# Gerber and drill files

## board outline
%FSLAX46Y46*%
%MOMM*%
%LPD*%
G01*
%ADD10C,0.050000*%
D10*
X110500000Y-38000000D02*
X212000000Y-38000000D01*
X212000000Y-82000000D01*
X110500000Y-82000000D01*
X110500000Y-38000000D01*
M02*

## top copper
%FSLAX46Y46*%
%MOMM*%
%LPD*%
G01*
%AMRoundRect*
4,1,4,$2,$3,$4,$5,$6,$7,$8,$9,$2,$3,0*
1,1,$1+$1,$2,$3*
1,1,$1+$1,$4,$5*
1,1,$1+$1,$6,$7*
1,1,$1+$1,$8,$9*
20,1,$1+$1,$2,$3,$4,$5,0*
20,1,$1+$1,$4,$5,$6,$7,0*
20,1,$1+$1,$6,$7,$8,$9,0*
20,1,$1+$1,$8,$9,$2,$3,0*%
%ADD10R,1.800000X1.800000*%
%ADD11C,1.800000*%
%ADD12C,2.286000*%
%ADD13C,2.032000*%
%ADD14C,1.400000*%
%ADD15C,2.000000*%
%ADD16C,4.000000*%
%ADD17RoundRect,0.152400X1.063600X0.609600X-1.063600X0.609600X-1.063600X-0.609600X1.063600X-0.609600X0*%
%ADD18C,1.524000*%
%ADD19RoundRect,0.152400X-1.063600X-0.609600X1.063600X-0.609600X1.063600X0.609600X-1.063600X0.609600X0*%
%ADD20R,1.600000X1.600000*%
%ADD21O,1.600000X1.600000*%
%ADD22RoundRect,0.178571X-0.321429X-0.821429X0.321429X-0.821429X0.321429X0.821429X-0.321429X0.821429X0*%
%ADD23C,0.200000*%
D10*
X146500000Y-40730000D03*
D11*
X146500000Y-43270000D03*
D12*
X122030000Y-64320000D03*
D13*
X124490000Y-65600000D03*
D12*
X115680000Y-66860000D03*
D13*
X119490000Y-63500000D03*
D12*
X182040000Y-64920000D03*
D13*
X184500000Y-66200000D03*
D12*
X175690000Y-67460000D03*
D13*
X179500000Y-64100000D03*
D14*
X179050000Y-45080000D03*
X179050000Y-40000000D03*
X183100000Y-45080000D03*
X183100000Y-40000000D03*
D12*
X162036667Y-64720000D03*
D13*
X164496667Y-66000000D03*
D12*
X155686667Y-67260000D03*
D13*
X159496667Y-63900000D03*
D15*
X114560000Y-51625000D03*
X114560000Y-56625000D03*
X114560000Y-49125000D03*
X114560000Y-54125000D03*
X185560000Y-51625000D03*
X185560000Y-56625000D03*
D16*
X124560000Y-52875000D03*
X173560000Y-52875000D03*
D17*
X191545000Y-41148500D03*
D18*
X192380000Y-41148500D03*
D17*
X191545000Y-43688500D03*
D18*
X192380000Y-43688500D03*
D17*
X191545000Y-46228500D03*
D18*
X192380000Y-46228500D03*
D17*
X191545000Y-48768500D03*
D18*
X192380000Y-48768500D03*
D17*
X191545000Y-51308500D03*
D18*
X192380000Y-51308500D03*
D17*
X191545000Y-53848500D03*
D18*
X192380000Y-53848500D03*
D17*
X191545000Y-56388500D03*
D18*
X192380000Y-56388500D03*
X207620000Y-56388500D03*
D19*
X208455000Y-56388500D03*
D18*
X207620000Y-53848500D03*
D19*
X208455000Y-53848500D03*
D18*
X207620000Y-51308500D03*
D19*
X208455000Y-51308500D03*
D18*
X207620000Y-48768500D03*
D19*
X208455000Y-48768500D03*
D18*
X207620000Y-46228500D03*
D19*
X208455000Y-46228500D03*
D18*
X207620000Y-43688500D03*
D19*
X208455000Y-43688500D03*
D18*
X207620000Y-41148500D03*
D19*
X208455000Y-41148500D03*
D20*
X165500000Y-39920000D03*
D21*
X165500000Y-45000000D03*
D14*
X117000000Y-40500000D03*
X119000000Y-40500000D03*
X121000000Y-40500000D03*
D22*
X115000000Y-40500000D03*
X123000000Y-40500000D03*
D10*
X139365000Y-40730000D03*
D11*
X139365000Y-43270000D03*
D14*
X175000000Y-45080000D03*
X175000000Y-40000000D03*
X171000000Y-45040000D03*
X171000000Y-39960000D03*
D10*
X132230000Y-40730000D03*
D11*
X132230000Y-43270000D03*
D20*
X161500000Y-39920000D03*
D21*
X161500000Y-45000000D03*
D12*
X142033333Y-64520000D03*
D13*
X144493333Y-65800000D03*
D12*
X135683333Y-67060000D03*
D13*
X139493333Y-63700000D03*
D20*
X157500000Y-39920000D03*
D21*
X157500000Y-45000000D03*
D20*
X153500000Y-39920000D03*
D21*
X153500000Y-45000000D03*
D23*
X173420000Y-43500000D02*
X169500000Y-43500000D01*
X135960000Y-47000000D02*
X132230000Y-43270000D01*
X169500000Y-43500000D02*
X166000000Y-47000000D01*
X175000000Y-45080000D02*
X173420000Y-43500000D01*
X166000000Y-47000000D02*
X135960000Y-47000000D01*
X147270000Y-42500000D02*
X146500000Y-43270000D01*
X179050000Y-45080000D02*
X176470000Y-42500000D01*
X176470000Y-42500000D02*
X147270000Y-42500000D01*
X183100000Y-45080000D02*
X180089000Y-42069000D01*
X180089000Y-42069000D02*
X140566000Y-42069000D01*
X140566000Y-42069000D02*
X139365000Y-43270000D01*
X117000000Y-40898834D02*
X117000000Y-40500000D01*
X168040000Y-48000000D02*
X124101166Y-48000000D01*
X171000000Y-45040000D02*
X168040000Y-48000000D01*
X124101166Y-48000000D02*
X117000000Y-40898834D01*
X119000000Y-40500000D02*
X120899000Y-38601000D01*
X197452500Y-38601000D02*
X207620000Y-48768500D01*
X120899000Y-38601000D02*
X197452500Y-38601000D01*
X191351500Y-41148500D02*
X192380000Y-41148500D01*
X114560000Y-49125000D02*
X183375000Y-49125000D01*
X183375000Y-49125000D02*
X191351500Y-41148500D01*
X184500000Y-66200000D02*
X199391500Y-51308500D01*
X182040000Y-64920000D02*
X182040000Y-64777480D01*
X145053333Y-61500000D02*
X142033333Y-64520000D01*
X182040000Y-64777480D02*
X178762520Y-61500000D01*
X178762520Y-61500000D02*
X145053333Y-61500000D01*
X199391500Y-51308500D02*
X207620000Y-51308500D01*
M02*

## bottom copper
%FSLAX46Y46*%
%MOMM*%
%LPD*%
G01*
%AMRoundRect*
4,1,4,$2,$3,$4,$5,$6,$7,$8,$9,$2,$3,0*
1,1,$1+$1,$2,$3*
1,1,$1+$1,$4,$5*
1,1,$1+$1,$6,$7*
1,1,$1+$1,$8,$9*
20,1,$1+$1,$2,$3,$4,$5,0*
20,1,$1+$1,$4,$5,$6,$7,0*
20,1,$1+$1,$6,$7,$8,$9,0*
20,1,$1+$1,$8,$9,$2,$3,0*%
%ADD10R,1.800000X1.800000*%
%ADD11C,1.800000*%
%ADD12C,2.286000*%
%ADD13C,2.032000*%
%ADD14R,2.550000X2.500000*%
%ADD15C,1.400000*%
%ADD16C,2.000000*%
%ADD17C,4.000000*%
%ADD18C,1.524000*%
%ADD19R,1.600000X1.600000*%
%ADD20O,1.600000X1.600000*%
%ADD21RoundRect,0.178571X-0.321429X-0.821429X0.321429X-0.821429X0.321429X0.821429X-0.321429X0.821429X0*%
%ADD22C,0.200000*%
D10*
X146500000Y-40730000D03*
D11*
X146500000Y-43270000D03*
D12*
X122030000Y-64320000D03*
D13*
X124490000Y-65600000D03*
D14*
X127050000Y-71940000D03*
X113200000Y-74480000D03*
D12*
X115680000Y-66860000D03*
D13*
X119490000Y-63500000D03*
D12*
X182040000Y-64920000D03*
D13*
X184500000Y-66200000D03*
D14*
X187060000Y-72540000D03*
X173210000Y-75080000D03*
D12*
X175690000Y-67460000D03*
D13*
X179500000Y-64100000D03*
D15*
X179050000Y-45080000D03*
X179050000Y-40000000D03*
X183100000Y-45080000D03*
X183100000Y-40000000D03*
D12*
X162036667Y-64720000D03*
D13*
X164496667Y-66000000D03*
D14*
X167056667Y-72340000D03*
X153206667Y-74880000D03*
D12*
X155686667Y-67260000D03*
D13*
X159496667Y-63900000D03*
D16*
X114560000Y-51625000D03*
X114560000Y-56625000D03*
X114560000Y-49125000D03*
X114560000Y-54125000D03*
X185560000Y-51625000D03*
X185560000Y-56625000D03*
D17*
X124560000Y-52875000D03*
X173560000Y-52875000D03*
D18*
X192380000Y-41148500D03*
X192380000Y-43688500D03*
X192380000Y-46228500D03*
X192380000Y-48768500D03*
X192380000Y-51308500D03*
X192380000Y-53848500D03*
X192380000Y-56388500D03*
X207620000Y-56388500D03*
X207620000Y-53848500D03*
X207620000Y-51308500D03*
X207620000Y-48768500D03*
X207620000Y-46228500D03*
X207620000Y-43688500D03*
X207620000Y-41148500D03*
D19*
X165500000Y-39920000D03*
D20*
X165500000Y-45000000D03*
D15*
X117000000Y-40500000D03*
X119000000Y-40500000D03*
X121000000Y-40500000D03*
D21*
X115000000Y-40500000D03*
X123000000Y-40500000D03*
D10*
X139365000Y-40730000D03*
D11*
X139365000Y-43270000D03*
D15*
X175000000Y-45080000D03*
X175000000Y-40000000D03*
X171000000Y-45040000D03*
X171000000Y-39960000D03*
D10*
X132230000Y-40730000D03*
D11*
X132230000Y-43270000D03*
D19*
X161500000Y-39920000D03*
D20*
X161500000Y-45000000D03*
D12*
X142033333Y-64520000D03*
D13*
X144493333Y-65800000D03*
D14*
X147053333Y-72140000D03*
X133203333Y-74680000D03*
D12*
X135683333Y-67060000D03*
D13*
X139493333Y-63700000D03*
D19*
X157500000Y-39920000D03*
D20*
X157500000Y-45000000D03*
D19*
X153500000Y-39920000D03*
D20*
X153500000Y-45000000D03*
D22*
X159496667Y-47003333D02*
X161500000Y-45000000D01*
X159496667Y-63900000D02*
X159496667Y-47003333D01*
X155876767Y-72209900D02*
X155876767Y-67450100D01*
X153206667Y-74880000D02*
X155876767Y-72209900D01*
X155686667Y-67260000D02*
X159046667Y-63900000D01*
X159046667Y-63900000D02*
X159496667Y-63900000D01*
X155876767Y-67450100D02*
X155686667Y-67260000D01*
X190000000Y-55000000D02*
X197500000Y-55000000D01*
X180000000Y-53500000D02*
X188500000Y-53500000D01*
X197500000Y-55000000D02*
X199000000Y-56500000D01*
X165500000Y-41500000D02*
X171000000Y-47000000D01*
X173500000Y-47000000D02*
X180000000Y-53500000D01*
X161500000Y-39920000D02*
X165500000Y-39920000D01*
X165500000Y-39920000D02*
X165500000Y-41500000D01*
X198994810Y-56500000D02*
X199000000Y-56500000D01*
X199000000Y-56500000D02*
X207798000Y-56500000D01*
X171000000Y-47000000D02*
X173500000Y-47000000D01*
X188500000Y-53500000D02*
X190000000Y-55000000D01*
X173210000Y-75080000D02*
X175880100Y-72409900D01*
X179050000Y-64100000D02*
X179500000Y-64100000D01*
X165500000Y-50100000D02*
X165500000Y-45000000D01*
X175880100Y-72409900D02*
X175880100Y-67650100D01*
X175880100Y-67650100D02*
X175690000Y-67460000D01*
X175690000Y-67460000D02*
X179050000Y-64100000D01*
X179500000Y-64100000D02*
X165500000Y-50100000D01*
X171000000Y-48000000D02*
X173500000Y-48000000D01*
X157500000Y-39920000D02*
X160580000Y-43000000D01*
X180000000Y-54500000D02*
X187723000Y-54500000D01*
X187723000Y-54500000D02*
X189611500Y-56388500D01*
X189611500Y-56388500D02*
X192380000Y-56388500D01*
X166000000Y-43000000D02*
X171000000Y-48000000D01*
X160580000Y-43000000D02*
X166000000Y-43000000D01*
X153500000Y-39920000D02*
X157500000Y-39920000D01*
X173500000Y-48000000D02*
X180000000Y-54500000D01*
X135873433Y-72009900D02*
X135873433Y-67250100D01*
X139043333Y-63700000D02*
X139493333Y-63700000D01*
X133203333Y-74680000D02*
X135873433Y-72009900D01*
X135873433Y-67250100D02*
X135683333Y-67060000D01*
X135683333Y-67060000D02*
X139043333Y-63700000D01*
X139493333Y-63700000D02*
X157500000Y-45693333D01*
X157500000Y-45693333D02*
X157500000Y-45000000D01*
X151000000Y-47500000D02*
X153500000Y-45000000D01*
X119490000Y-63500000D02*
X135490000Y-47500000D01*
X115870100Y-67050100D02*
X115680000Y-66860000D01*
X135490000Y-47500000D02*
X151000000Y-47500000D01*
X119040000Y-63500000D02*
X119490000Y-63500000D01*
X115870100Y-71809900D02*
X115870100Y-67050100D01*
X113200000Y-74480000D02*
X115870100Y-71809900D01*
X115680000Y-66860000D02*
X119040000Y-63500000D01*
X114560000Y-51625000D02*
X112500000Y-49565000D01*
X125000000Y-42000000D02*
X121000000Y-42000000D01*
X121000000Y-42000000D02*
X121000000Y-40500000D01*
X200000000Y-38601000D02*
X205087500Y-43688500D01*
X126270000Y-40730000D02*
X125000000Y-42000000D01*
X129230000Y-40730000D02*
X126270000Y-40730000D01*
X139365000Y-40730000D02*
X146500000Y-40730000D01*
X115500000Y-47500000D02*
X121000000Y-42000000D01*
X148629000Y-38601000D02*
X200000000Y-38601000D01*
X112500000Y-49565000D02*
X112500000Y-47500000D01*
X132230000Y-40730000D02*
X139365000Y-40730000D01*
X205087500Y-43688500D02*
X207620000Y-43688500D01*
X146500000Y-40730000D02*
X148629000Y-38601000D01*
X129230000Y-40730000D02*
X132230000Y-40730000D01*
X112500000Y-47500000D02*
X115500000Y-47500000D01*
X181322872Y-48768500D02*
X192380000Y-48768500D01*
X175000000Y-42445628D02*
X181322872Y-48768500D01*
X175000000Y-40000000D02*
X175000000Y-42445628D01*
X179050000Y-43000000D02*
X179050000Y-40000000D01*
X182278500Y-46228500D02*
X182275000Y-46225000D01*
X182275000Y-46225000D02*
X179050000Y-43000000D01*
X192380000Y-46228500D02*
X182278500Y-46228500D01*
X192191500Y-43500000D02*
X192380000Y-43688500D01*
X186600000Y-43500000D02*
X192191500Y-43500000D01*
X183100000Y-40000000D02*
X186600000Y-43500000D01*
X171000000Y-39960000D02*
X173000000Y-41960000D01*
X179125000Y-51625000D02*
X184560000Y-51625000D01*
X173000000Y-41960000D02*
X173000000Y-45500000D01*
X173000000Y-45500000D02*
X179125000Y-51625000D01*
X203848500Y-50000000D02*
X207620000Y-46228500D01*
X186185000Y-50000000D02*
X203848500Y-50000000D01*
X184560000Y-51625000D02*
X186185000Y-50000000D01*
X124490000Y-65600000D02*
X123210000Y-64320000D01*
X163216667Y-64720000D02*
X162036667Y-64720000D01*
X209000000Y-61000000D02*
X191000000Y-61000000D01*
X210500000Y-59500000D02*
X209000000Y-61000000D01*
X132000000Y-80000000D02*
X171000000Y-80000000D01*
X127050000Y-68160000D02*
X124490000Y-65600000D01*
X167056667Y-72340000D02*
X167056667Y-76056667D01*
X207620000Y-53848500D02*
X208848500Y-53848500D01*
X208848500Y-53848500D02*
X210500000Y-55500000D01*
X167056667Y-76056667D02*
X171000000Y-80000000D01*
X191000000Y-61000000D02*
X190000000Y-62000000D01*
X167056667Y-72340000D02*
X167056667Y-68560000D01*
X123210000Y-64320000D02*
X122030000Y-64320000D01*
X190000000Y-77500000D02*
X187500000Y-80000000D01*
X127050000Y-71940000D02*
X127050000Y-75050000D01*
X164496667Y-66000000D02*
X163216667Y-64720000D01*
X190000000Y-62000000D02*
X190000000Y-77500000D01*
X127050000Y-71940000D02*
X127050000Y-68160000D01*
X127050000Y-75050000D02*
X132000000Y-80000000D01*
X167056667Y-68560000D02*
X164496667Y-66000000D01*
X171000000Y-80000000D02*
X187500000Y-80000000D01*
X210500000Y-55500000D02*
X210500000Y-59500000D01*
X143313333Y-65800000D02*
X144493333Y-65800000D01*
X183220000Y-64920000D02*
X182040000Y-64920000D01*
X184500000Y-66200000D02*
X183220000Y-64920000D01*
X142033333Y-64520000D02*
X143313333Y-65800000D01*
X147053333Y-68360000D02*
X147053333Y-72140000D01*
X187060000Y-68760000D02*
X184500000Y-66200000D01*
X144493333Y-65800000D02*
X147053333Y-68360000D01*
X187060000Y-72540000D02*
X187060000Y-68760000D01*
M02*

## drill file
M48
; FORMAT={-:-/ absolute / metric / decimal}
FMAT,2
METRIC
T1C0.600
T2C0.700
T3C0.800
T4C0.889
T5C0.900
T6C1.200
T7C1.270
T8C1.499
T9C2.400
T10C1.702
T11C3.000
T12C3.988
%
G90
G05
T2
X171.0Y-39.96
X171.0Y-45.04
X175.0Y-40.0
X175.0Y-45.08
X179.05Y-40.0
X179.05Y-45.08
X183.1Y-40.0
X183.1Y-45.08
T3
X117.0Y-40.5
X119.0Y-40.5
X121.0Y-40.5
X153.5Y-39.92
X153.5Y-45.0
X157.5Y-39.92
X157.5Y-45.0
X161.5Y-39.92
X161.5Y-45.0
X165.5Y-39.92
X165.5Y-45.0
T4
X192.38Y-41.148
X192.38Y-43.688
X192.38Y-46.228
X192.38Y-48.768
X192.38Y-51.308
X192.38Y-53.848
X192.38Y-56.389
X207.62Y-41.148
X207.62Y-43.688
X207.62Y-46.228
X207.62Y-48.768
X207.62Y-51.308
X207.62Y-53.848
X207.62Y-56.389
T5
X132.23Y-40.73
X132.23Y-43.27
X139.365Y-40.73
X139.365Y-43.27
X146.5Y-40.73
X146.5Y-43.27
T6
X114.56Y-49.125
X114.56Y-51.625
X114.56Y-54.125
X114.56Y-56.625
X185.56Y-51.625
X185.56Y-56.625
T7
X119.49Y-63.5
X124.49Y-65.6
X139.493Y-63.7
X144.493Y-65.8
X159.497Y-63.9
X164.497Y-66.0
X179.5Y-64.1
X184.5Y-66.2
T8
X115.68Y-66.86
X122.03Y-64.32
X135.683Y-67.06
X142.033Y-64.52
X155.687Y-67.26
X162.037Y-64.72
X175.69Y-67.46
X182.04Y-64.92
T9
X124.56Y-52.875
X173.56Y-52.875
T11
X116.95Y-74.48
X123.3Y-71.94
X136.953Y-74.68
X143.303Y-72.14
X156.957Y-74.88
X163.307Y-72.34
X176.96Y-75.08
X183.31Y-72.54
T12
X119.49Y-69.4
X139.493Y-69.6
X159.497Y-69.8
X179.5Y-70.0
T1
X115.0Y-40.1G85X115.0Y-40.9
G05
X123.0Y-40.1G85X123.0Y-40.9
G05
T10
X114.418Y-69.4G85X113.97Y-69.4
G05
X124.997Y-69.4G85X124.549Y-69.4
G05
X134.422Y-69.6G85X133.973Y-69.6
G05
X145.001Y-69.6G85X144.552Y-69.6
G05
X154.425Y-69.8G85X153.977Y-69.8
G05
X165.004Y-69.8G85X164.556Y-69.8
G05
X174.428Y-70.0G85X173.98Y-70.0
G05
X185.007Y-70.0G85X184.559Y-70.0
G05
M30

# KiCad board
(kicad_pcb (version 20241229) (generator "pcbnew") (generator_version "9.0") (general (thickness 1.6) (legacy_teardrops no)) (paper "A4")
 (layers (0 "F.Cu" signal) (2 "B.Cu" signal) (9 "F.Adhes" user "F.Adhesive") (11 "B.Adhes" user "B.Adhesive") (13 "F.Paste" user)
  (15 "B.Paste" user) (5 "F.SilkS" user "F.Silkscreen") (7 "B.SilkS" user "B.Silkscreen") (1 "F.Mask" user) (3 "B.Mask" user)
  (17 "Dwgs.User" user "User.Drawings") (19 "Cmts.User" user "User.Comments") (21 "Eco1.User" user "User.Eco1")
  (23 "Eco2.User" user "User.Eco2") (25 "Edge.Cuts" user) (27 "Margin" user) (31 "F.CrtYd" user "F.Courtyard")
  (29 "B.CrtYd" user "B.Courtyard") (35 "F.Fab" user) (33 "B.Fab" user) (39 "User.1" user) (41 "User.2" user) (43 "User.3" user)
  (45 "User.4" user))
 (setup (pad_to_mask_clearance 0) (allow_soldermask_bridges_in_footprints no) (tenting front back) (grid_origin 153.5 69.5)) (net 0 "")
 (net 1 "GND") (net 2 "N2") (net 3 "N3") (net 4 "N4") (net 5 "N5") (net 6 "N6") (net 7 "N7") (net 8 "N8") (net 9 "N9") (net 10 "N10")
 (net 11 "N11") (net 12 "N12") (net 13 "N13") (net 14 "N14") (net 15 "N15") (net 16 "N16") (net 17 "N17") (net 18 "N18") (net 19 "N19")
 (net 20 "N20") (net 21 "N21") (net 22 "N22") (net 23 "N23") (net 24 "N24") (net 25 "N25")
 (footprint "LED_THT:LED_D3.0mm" (layer "F.Cu") (at 146.5 40.73 -90)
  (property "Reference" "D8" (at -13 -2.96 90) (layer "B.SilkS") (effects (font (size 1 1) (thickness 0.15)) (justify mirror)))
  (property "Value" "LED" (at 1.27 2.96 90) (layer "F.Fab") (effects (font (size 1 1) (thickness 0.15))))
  (pad "1" thru_hole rect (at 0 0 270) (size 1.8 1.8) (drill 0.9) (layers "*.Cu" "*.Mask") (remove_unused_layers no) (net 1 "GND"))
  (pad "2" thru_hole circle (at 2.54 0 270) (size 1.8 1.8) (drill 0.9) (layers "*.Cu" "*.Mask") (remove_unused_layers no) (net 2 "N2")))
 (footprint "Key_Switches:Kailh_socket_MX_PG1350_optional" (layer "F.Cu") (at 119.49 69.4)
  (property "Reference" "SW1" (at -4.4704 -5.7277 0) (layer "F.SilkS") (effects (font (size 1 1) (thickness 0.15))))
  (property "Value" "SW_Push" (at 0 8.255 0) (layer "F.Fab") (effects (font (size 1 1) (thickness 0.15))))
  (pad "" np_thru_hole oval (at -5.2959 0 180) (size 2.15 1.7018) (drill oval 2.15 1.7018) (layers "*.Cu" "*.Mask"))
  (pad "" np_thru_hole circle (at -2.54 5.08) (size 3 3) (drill 3) (layers "*.Cu" "*.Mask"))
  (pad "" np_thru_hole circle (at 0 0) (size 3.9878 3.9878) (drill 3.9878) (layers "*.Cu" "*.Mask"))
  (pad "" np_thru_hole circle (at 3.81 2.54) (size 3 3) (drill 3) (layers "*.Cu" "*.Mask"))
  (pad "" np_thru_hole oval (at 5.2832 0 180) (size 2.15 1.7018) (drill oval 2.15 1.7018) (layers "*.Cu" "*.Mask"))
  (pad "1" thru_hole circle (at 2.54 -5.08) (size 2.286 2.286) (drill 1.4986) (layers "*.Cu" "*.Mask") (remove_unused_layers no)
   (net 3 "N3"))
  (pad "1" thru_hole circle (at 5 -3.8 180) (size 2.032 2.032) (drill 1.27) (layers "*.Cu" "*.Mask") (remove_unused_layers no) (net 3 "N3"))
  (pad "1" smd rect (at 7.56 2.54) (size 2.55 2.5) (layers "B.Cu" "B.Mask" "B.Paste") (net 3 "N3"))
  (pad "2" smd rect (at -6.29 5.08) (size 2.55 2.5) (layers "B.Cu" "B.Mask" "B.Paste") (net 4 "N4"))
  (pad "2" thru_hole circle (at -3.81 -2.54) (size 2.286 2.286) (drill 1.4986) (layers "*.Cu" "*.Mask") (remove_unused_layers no)
   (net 4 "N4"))
  (pad "2" thru_hole circle (at 0 -5.9 180) (size 2.032 2.032) (drill 1.27) (layers "*.Cu" "*.Mask") (remove_unused_layers no) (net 4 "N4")))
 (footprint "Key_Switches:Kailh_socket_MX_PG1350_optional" (layer "F.Cu") (at 179.5 70)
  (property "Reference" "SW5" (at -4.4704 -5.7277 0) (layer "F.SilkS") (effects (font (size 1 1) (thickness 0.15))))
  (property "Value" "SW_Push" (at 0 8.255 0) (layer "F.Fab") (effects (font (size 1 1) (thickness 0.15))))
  (pad "" np_thru_hole oval (at -5.2959 0 180) (size 2.15 1.7018) (drill oval 2.15 1.7018) (layers "*.Cu" "*.Mask"))
  (pad "" np_thru_hole circle (at -2.54 5.08) (size 3 3) (drill 3) (layers "*.Cu" "*.Mask"))
  (pad "" np_thru_hole circle (at 0 0) (size 3.9878 3.9878) (drill 3.9878) (layers "*.Cu" "*.Mask"))
  (pad "" np_thru_hole circle (at 3.81 2.54) (size 3 3) (drill 3) (layers "*.Cu" "*.Mask"))
  (pad "" np_thru_hole oval (at 5.2832 0 180) (size 2.15 1.7018) (drill oval 2.15 1.7018) (layers "*.Cu" "*.Mask"))
  (pad "1" thru_hole circle (at 2.54 -5.08) (size 2.286 2.286) (drill 1.4986) (layers "*.Cu" "*.Mask") (remove_unused_layers no)
   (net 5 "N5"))
  (pad "1" thru_hole circle (at 5 -3.8 180) (size 2.032 2.032) (drill 1.27) (layers "*.Cu" "*.Mask") (remove_unused_layers no) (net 5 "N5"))
  (pad "1" smd rect (at 7.56 2.54) (size 2.55 2.5) (layers "B.Cu" "B.Mask" "B.Paste") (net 5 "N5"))
  (pad "2" smd rect (at -6.29 5.08) (size 2.55 2.5) (layers "B.Cu" "B.Mask" "B.Paste") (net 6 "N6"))
  (pad "2" thru_hole circle (at -3.81 -2.54) (size 2.286 2.286) (drill 1.4986) (layers "*.Cu" "*.Mask") (remove_unused_layers no)
   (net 6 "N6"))
  (pad "2" thru_hole circle (at 0 -5.9 180) (size 2.032 2.032) (drill 1.27) (layers "*.Cu" "*.Mask") (remove_unused_layers no) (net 6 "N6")))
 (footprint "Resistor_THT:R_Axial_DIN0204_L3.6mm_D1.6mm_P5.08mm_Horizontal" (layer "F.Cu") (at 179.05 45.08 90)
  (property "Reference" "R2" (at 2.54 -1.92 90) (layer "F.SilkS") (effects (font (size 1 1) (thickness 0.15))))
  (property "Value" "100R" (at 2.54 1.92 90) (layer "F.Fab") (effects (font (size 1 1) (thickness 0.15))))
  (pad "1" thru_hole circle (at 0 0 90) (size 1.4 1.4) (drill 0.7) (layers "*.Cu" "*.Mask") (remove_unused_layers no) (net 2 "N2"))
  (pad "2" thru_hole circle (at 5.08 0 90) (size 1.4 1.4) (drill 0.7) (layers "*.Cu" "*.Mask") (remove_unused_layers no) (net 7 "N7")))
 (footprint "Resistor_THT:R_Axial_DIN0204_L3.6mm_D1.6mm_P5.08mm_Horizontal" (layer "F.Cu") (at 183.1 45.08 90)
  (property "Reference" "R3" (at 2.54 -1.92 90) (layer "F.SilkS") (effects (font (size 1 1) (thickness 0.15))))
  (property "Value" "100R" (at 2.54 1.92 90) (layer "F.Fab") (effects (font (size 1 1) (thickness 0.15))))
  (pad "1" thru_hole circle (at 0 0 90) (size 1.4 1.4) (drill 0.7) (layers "*.Cu" "*.Mask") (remove_unused_layers no) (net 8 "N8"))
  (pad "2" thru_hole circle (at 5.08 0 90) (size 1.4 1.4) (drill 0.7) (layers "*.Cu" "*.Mask") (remove_unused_layers no) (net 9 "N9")))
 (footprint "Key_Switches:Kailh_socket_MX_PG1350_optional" (layer "F.Cu") (at 159.496667 69.8)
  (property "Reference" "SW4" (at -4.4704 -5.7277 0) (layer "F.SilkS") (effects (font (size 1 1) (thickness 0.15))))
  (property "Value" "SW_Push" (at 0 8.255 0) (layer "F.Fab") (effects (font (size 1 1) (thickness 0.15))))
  (pad "" np_thru_hole oval (at -5.2959 0 180) (size 2.15 1.7018) (drill oval 2.15 1.7018) (layers "*.Cu" "*.Mask"))
  (pad "" np_thru_hole circle (at -2.54 5.08) (size 3 3) (drill 3) (layers "*.Cu" "*.Mask"))
  (pad "" np_thru_hole circle (at 0 0) (size 3.9878 3.9878) (drill 3.9878) (layers "*.Cu" "*.Mask"))
  (pad "" np_thru_hole circle (at 3.81 2.54) (size 3 3) (drill 3) (layers "*.Cu" "*.Mask"))
  (pad "" np_thru_hole oval (at 5.2832 0 180) (size 2.15 1.7018) (drill oval 2.15 1.7018) (layers "*.Cu" "*.Mask"))
  (pad "1" thru_hole circle (at 2.54 -5.08) (size 2.286 2.286) (drill 1.4986) (layers "*.Cu" "*.Mask") (remove_unused_layers no)
   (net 3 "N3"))
  (pad "1" thru_hole circle (at 5 -3.8 180) (size 2.032 2.032) (drill 1.27) (layers "*.Cu" "*.Mask") (remove_unused_layers no) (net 3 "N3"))
  (pad "1" smd rect (at 7.56 2.54) (size 2.55 2.5) (layers "B.Cu" "B.Mask" "B.Paste") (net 3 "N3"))
  (pad "2" smd rect (at -6.29 5.08) (size 2.55 2.5) (layers "B.Cu" "B.Mask" "B.Paste") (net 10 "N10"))
  (pad "2" thru_hole circle (at -3.81 -2.54) (size 2.286 2.286) (drill 1.4986) (layers "*.Cu" "*.Mask") (remove_unused_layers no)
   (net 10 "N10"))
  (pad "2" thru_hole circle (at 0 -5.9 180) (size 2.032 2.032) (drill 1.27) (layers "*.Cu" "*.Mask") (remove_unused_layers no)
   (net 10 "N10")))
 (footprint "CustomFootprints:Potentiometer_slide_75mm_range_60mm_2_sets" (layer "F.Cu") (at 112.06 57.625)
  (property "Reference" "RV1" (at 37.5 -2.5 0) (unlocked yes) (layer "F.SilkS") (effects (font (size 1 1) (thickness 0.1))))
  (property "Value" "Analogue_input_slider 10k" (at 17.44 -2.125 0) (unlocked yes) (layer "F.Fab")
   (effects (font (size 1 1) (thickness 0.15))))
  (pad "1" thru_hole circle (at 2.5 -6) (size 2 2) (drill 1.2) (layers "*.Cu" "*.Mask") (remove_unused_layers no) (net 1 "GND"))
  (pad "1'" thru_hole circle (at 2.5 -1) (size 2 2) (drill 1.2) (layers "*.Cu" "*.Mask") (remove_unused_layers no))
  (pad "2" thru_hole circle (at 2.5 -8.5) (size 2 2) (drill 1.2) (layers "*.Cu" "*.Mask") (remove_unused_layers no) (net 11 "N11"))
  (pad "2'" thru_hole circle (at 2.5 -3.5) (size 2 2) (drill 1.2) (layers "*.Cu" "*.Mask") (remove_unused_layers no))
  (pad "3" thru_hole circle (at 73.5 -6) (size 2 2) (drill 1.2) (layers "*.Cu" "*.Mask") (remove_unused_layers no) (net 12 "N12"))
  (pad "3'" thru_hole circle (at 73.5 -1) (size 2 2) (drill 1.2) (layers "*.Cu" "*.Mask") (remove_unused_layers no))
  (pad "MP" thru_hole circle (at 12.5 -4.75) (size 4 4) (drill 2.4) (layers "*.Cu" "*.Mask") (remove_unused_layers no))
  (pad "MP" thru_hole circle (at 61.5 -4.75) (size 4 4) (drill 2.4) (layers "*.Cu" "*.Mask") (remove_unused_layers no)))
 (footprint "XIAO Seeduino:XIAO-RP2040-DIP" (layer "F.Cu") (at 200 48.7685)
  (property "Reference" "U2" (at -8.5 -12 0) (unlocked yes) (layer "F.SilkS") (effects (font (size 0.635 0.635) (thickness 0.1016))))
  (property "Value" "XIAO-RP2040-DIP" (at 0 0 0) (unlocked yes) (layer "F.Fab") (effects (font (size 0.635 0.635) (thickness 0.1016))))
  (pad "1" smd roundrect (at -8.455 -7.62 180) (size 2.432 1.524) (layers "F.Cu" "F.Mask") (roundrect_rratio 0.1) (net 11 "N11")
   (thermal_bridge_angle 45))
  (pad "1" thru_hole circle (at -7.62 -7.62 180) (size 1.524 1.524) (drill 0.889) (layers "*.Cu" "*.Mask") (remove_unused_layers no)
   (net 11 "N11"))
  (pad "2" smd roundrect (at -8.455 -5.08 180) (size 2.432 1.524) (layers "F.Cu" "F.Mask") (roundrect_rratio 0.1) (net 9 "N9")
   (thermal_bridge_angle 45))
  (pad "2" thru_hole circle (at -7.62 -5.08 180) (size 1.524 1.524) (drill 0.889) (layers "*.Cu" "*.Mask") (remove_unused_layers no)
   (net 9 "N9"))
  (pad "3" smd roundrect (at -8.455 -2.54 180) (size 2.432 1.524) (layers "F.Cu" "F.Mask") (roundrect_rratio 0.1) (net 7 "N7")
   (thermal_bridge_angle 45))
  (pad "3" thru_hole circle (at -7.62 -2.54 180) (size 1.524 1.524) (drill 0.889) (layers "*.Cu" "*.Mask") (remove_unused_layers no)
   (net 7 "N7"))
  (pad "4" smd roundrect (at -8.455 0 180) (size 2.432 1.524) (layers "F.Cu" "F.Mask") (roundrect_rratio 0.1) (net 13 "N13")
   (thermal_bridge_angle 45))
  (pad "4" thru_hole circle (at -7.62 0 180) (size 1.524 1.524) (drill 0.889) (layers "*.Cu" "*.Mask") (remove_unused_layers no)
   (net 13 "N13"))
  (pad "5" smd roundrect (at -8.455 2.54 180) (size 2.432 1.524) (layers "F.Cu" "F.Mask") (roundrect_rratio 0.1) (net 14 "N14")
   (thermal_bridge_angle 45))
  (pad "5" thru_hole circle (at -7.62 2.54 180) (size 1.524 1.524) (drill 0.889) (layers "*.Cu" "*.Mask") (remove_unused_layers no)
   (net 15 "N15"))
  (pad "6" smd roundrect (at -8.455 5.08 180) (size 2.432 1.524) (layers "F.Cu" "F.Mask") (roundrect_rratio 0.1) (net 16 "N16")
   (thermal_bridge_angle 45))
  (pad "6" thru_hole circle (at -7.62 5.08 180) (size 1.524 1.524) (drill 0.889) (layers "*.Cu" "*.Mask") (remove_unused_layers no)
   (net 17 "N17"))
  (pad "7" smd roundrect (at -8.455 7.62 180) (size 2.432 1.524) (layers "F.Cu" "F.Mask") (roundrect_rratio 0.1) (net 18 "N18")
   (thermal_bridge_angle 45))
  (pad "7" thru_hole circle (at -7.62 7.62 180) (size 1.524 1.524) (drill 0.889) (layers "*.Cu" "*.Mask") (remove_unused_layers no)
   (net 18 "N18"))
  (pad "8" thru_hole circle (at 7.62 7.62) (size 1.524 1.524) (drill 0.889) (layers "*.Cu" "*.Mask") (remove_unused_layers no)
   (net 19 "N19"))
  (pad "8" smd roundrect (at 8.455 7.62) (size 2.432 1.524) (layers "F.Cu" "F.Mask") (roundrect_rratio 0.1) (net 19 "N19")
   (thermal_bridge_angle 45))
  (pad "9" thru_hole circle (at 7.62 5.08) (size 1.524 1.524) (drill 0.889) (layers "*.Cu" "*.Mask") (remove_unused_layers no) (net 3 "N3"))
  (pad "9" smd roundrect (at 8.455 5.08) (size 2.432 1.524) (layers "F.Cu" "F.Mask") (roundrect_rratio 0.1) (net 3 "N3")
   (thermal_bridge_angle 45))
  (pad "10" thru_hole circle (at 7.62 2.54) (size 1.524 1.524) (drill 0.889) (layers "*.Cu" "*.Mask") (remove_unused_layers no) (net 5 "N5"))
  (pad "10" smd roundrect (at 8.455 2.54) (size 2.432 1.524) (layers "F.Cu" "F.Mask") (roundrect_rratio 0.1) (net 5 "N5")
   (thermal_bridge_angle 45))
  (pad "11" thru_hole circle (at 7.62 0) (size 1.524 1.524) (drill 0.889) (layers "*.Cu" "*.Mask") (remove_unused_layers no) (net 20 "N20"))
  (pad "11" smd roundrect (at 8.455 0) (size 2.432 1.524) (layers "F.Cu" "F.Mask") (roundrect_rratio 0.1) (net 20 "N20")
   (thermal_bridge_angle 45))
  (pad "12" thru_hole circle (at 7.62 -2.54) (size 1.524 1.524) (drill 0.889) (layers "*.Cu" "*.Mask") (remove_unused_layers no)
   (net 12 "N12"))
  (pad "12" smd roundrect (at 8.455 -2.54) (size 2.432 1.524) (layers "F.Cu" "F.Mask") (roundrect_rratio 0.1) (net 12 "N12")
   (thermal_bridge_angle 45))
  (pad "13" thru_hole circle (at 7.62 -5.08) (size 1.524 1.524) (drill 0.889) (layers "*.Cu" "*.Mask") (remove_unused_layers no)
   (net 1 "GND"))
  (pad "13" smd roundrect (at 8.455 -5.08) (size 2.432 1.524) (layers "F.Cu" "F.Mask") (roundrect_rratio 0.1) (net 1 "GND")
   (thermal_bridge_angle 45))
  (pad "14" thru_hole circle (at 7.62 -7.62) (size 1.524 1.524) (drill 0.889) (layers "*.Cu" "*.Mask") (remove_unused_layers no)
   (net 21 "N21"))
  (pad "14" smd roundrect (at 8.455 -7.62) (size 2.432 1.524) (layers "F.Cu" "F.Mask") (roundrect_rratio 0.1) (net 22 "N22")
   (thermal_bridge_angle 45)))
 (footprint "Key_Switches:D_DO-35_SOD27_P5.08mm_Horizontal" (layer "F.Cu") (at 165.5 38.65 -90)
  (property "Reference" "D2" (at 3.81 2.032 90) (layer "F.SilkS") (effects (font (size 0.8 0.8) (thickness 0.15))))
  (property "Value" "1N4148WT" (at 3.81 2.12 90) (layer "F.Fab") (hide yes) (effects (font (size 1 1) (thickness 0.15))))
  (pad "1" thru_hole rect (at 1.27 0 270) (size 1.6 1.6) (drill 0.8) (layers "*.Cu" "*.Mask") (remove_unused_layers no) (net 19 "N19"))
  (pad "2" thru_hole oval (at 6.35 0 270) (size 1.6 1.6) (drill 0.8) (layers "*.Cu" "*.Mask") (remove_unused_layers no) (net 6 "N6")))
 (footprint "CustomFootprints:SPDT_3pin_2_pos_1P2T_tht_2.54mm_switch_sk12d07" (layer "F.Cu") (at 114.7 38.25)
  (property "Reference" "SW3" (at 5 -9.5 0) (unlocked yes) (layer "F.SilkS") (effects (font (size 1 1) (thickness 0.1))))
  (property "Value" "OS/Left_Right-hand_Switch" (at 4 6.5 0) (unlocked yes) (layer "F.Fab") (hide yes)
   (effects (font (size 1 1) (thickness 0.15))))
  (pad "1" thru_hole circle (at 2.3 2.25) (size 1.4 1.4) (drill 0.8) (layers "*.Cu" "*.Mask") (remove_unused_layers no) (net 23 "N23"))
  (pad "2" thru_hole circle (at 4.3 2.25) (size 1.4 1.4) (drill 0.8) (layers "*.Cu" "*.Mask") (remove_unused_layers no) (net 20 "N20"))
  (pad "3" thru_hole circle (at 6.3 2.25) (size 1.4 1.4) (drill 0.8) (layers "*.Cu" "*.Mask") (remove_unused_layers no) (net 1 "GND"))
  (pad "MH" thru_hole roundrect (at 0.3 2.25) (size 1 2) (drill oval 0.6 1.4) (layers "*.Cu" "*.Mask") (remove_unused_layers no)
   (roundrect_rratio 0.1785714286))
  (pad "MH" thru_hole roundrect (at 8.3 2.25) (size 1 2) (drill oval 0.6 1.4) (layers "*.Cu" "*.Mask") (remove_unused_layers no)
   (roundrect_rratio 0.1785714286)))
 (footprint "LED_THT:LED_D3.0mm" (layer "F.Cu") (at 139.365 40.73 -90)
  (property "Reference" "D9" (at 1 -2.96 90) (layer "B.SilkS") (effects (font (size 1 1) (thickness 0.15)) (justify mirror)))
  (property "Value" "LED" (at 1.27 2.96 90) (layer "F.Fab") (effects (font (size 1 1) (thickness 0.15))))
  (pad "1" thru_hole rect (at 0 0 270) (size 1.8 1.8) (drill 0.9) (layers "*.Cu" "*.Mask") (remove_unused_layers no) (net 1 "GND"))
  (pad "2" thru_hole circle (at 2.54 0 270) (size 1.8 1.8) (drill 0.9) (layers "*.Cu" "*.Mask") (remove_unused_layers no) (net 8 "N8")))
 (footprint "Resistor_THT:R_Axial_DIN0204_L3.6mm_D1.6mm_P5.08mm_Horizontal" (layer "F.Cu") (at 175 45.08 90)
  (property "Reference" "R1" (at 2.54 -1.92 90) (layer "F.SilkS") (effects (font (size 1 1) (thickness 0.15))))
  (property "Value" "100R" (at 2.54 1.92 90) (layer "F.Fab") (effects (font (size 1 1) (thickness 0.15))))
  (pad "1" thru_hole circle (at 0 0 90) (size 1.4 1.4) (drill 0.7) (layers "*.Cu" "*.Mask") (remove_unused_layers no) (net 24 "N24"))
  (pad "2" thru_hole circle (at 5.08 0 90) (size 1.4 1.4) (drill 0.7) (layers "*.Cu" "*.Mask") (remove_unused_layers no) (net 13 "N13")))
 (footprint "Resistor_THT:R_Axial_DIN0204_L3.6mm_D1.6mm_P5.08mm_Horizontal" (layer "F.Cu") (at 171 45.04 90)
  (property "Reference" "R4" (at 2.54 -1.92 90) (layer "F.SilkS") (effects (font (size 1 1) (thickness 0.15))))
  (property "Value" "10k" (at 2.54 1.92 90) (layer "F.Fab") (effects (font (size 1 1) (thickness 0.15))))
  (pad "1" thru_hole circle (at 0 0 90) (size 1.4 1.4) (drill 0.7) (layers "*.Cu" "*.Mask") (remove_unused_layers no) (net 23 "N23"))
  (pad "2" thru_hole circle (at 5.08 0 90) (size 1.4 1.4) (drill 0.7) (layers "*.Cu" "*.Mask") (remove_unused_layers no) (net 12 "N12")))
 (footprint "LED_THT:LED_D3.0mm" (layer "F.Cu") (at 132.23 40.73 -90)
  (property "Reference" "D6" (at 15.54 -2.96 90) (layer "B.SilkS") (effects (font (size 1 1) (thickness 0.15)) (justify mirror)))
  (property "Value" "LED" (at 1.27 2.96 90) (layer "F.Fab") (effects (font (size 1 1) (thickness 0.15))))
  (pad "1" thru_hole rect (at 0 0 270) (size 1.8 1.8) (drill 0.9) (layers "*.Cu" "*.Mask") (remove_unused_layers no) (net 1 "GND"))
  (pad "2" thru_hole circle (at 2.54 0 270) (size 1.8 1.8) (drill 0.9) (layers "*.Cu" "*.Mask") (remove_unused_layers no) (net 24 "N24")))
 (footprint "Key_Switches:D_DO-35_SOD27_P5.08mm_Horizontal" (layer "F.Cu") (at 161.5 38.65 -90)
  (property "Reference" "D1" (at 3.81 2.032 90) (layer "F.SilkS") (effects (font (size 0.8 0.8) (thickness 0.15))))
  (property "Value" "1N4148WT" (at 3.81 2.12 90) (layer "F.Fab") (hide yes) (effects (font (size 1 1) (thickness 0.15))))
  (pad "1" thru_hole rect (at 1.27 0 270) (size 1.6 1.6) (drill 0.8) (layers "*.Cu" "*.Mask") (remove_unused_layers no) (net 19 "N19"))
  (pad "2" thru_hole oval (at 6.35 0 270) (size 1.6 1.6) (drill 0.8) (layers "*.Cu" "*.Mask") (remove_unused_layers no) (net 10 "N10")))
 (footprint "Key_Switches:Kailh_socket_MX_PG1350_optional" (layer "F.Cu") (at 139.493333 69.6)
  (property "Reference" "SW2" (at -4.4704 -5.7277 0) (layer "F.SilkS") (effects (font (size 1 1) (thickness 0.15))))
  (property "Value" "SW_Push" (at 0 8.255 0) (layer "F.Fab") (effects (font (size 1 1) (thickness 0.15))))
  (pad "" np_thru_hole oval (at -5.2959 0 180) (size 2.15 1.7018) (drill oval 2.15 1.7018) (layers "*.Cu" "*.Mask"))
  (pad "" np_thru_hole circle (at -2.54 5.08) (size 3 3) (drill 3) (layers "*.Cu" "*.Mask"))
  (pad "" np_thru_hole circle (at 0 0) (size 3.9878 3.9878) (drill 3.9878) (layers "*.Cu" "*.Mask"))
  (pad "" np_thru_hole circle (at 3.81 2.54) (size 3 3) (drill 3) (layers "*.Cu" "*.Mask"))
  (pad "" np_thru_hole oval (at 5.2832 0 180) (size 2.15 1.7018) (drill oval 2.15 1.7018) (layers "*.Cu" "*.Mask"))
  (pad "1" thru_hole circle (at 2.54 -5.08) (size 2.286 2.286) (drill 1.4986) (layers "*.Cu" "*.Mask") (remove_unused_layers no)
   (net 5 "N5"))
  (pad "1" thru_hole circle (at 5 -3.8 180) (size 2.032 2.032) (drill 1.27) (layers "*.Cu" "*.Mask") (remove_unused_layers no) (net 5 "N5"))
  (pad "1" smd rect (at 7.56 2.54) (size 2.55 2.5) (layers "B.Cu" "B.Mask" "B.Paste") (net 5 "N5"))
  (pad "2" smd rect (at -6.29 5.08) (size 2.55 2.5) (layers "B.Cu" "B.Mask" "B.Paste") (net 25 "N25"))
  (pad "2" thru_hole circle (at -3.81 -2.54) (size 2.286 2.286) (drill 1.4986) (layers "*.Cu" "*.Mask") (remove_unused_layers no)
   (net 25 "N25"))
  (pad "2" thru_hole circle (at 0 -5.9 180) (size 2.032 2.032) (drill 1.27) (layers "*.Cu" "*.Mask") (remove_unused_layers no)
   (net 25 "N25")))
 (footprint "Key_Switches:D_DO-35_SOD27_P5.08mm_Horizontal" (layer "F.Cu") (at 157.5 38.65 -90)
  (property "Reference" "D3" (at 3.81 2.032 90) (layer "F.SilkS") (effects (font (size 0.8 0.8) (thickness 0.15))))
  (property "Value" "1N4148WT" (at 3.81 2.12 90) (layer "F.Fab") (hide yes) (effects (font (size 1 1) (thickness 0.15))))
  (pad "1" thru_hole rect (at 1.27 0 270) (size 1.6 1.6) (drill 0.8) (layers "*.Cu" "*.Mask") (remove_unused_layers no) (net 18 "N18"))
  (pad "2" thru_hole oval (at 6.35 0 270) (size 1.6 1.6) (drill 0.8) (layers "*.Cu" "*.Mask") (remove_unused_layers no) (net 25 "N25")))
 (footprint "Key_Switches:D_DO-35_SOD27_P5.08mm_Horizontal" (layer "F.Cu") (at 153.5 38.65 -90)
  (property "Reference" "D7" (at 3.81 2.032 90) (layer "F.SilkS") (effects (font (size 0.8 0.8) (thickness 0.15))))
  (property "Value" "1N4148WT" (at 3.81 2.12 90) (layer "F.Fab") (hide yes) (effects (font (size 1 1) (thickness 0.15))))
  (pad "1" thru_hole rect (at 1.27 0 270) (size 1.6 1.6) (drill 0.8) (layers "*.Cu" "*.Mask") (remove_unused_layers no) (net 18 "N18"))
  (pad "2" thru_hole oval (at 6.35 0 270) (size 1.6 1.6) (drill 0.8) (layers "*.Cu" "*.Mask") (remove_unused_layers no) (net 4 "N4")))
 (gr_rect (start 110.5 38) (end 212 82) (stroke (width 0.05) (type default)) (fill no) (layer "Edge.Cuts"))
 (segment (start 159.496667 47.003333) (end 161.5 45) (width 0.2) (layer "B.Cu") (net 10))
 (segment (start 159.496667 63.9) (end 159.496667 47.003333) (width 0.2) (layer "B.Cu") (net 10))
 (segment (start 155.876767 72.2099) (end 155.876767 67.4501) (width 0.2) (layer "B.Cu") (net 10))
 (segment (start 153.206667 74.88) (end 155.876767 72.2099) (width 0.2) (layer "B.Cu") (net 10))
 (segment (start 155.686667 67.26) (end 159.046667 63.9) (width 0.2) (layer "B.Cu") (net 10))
 (segment (start 159.046667 63.9) (end 159.496667 63.9) (width 0.2) (layer "B.Cu") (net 10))
 (segment (start 155.876767 67.4501) (end 155.686667 67.26) (width 0.2) (layer "B.Cu") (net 10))
 (segment (start 190 55) (end 197.5 55) (width 0.2) (layer "B.Cu") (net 19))
 (segment (start 180 53.5) (end 188.5 53.5) (width 0.2) (layer "B.Cu") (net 19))
 (segment (start 197.5 55) (end 199 56.5) (width 0.2) (layer "B.Cu") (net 19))
 (segment (start 165.5 41.5) (end 171 47) (width 0.2) (layer "B.Cu") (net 19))
 (segment (start 173.5 47) (end 180 53.5) (width 0.2) (layer "B.Cu") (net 19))
 (segment (start 161.5 39.92) (end 165.5 39.92) (width 0.2) (layer "B.Cu") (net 19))
 (segment (start 165.5 39.92) (end 165.5 41.5) (width 0.2) (layer "B.Cu") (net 19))
 (segment (start 198.99481 56.5) (end 199 56.5) (width 0.2) (layer "B.Cu") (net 19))
 (segment (start 199 56.5) (end 207.798 56.5) (width 0.2) (layer "B.Cu") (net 19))
 (segment (start 171 47) (end 173.5 47) (width 0.2) (layer "B.Cu") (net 19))
 (segment (start 188.5 53.5) (end 190 55) (width 0.2) (layer "B.Cu") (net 19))
 (segment (start 173.21 75.08) (end 175.8801 72.4099) (width 0.2) (layer "B.Cu") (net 6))
 (segment (start 179.05 64.1) (end 179.5 64.1) (width 0.2) (layer "B.Cu") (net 6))
 (segment (start 165.5 50.1) (end 165.5 45) (width 0.2) (layer "B.Cu") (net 6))
 (segment (start 175.8801 72.4099) (end 175.8801 67.6501) (width 0.2) (layer "B.Cu") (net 6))
 (segment (start 175.8801 67.6501) (end 175.69 67.46) (width 0.2) (layer "B.Cu") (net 6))
 (segment (start 175.69 67.46) (end 179.05 64.1) (width 0.2) (layer "B.Cu") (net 6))
 (segment (start 179.5 64.1) (end 165.5 50.1) (width 0.2) (layer "B.Cu") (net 6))
 (segment (start 171 48) (end 173.5 48) (width 0.2) (layer "B.Cu") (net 18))
 (segment (start 157.5 39.92) (end 160.58 43) (width 0.2) (layer "B.Cu") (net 18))
 (segment (start 180 54.5) (end 187.723 54.5) (width 0.2) (layer "B.Cu") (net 18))
 (segment (start 187.723 54.5) (end 189.6115 56.3885) (width 0.2) (layer "B.Cu") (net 18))
 (segment (start 189.6115 56.3885) (end 192.38 56.3885) (width 0.2) (layer "B.Cu") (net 18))
 (segment (start 166 43) (end 171 48) (width 0.2) (layer "B.Cu") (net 18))
 (segment (start 160.58 43) (end 166 43) (width 0.2) (layer "B.Cu") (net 18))
 (segment (start 153.5 39.92) (end 157.5 39.92) (width 0.2) (layer "B.Cu") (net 18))
 (segment (start 173.5 48) (end 180 54.5) (width 0.2) (layer "B.Cu") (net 18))
 (segment (start 135.873433 72.0099) (end 135.873433 67.2501) (width 0.2) (layer "B.Cu") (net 25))
 (segment (start 139.043333 63.7) (end 139.493333 63.7) (width 0.2) (layer "B.Cu") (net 25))
 (segment (start 133.203333 74.68) (end 135.873433 72.0099) (width 0.2) (layer "B.Cu") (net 25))
 (segment (start 135.873433 67.2501) (end 135.683333 67.06) (width 0.2) (layer "B.Cu") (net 25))
 (segment (start 135.683333 67.06) (end 139.043333 63.7) (width 0.2) (layer "B.Cu") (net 25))
 (segment (start 139.493333 63.7) (end 157.5 45.693333) (width 0.2) (layer "B.Cu") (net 25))
 (segment (start 157.5 45.693333) (end 157.5 45) (width 0.2) (layer "B.Cu") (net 25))
 (segment (start 151 47.5) (end 153.5 45) (width 0.2) (layer "B.Cu") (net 4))
 (segment (start 119.49 63.5) (end 135.49 47.5) (width 0.2) (layer "B.Cu") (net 4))
 (segment (start 115.8701 67.0501) (end 115.68 66.86) (width 0.2) (layer "B.Cu") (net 4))
 (segment (start 135.49 47.5) (end 151 47.5) (width 0.2) (layer "B.Cu") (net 4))
 (segment (start 119.04 63.5) (end 119.49 63.5) (width 0.2) (layer "B.Cu") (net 4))
 (segment (start 115.8701 71.8099) (end 115.8701 67.0501) (width 0.2) (layer "B.Cu") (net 4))
 (segment (start 113.2 74.48) (end 115.8701 71.8099) (width 0.2) (layer "B.Cu") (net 4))
 (segment (start 115.68 66.86) (end 119.04 63.5) (width 0.2) (layer "B.Cu") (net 4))
 (segment (start 173.42 43.5) (end 169.5 43.5) (width 0.2) (layer "F.Cu") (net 24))
 (segment (start 135.96 47) (end 132.23 43.27) (width 0.2) (layer "F.Cu") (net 24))
 (segment (start 169.5 43.5) (end 166 47) (width 0.2) (layer "F.Cu") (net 24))
 (segment (start 175 45.08) (end 173.42 43.5) (width 0.2) (layer "F.Cu") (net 24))
 (segment (start 166 47) (end 135.96 47) (width 0.2) (layer "F.Cu") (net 24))
 (segment (start 114.56 51.625) (end 112.5 49.565) (width 0.2) (layer "B.Cu") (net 1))
 (segment (start 125 42) (end 121 42) (width 0.2) (layer "B.Cu") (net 1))
 (segment (start 121 42) (end 121 40.5) (width 0.2) (layer "B.Cu") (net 1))
 (segment (start 200 38.601) (end 205.0875 43.6885) (width 0.2) (layer "B.Cu") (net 1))
 (segment (start 126.27 40.73) (end 125 42) (width 0.2) (layer "B.Cu") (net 1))
 (segment (start 129.23 40.73) (end 126.27 40.73) (width 0.2) (layer "B.Cu") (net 1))
 (segment (start 139.365 40.73) (end 146.5 40.73) (width 0.2) (layer "B.Cu") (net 1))
 (segment (start 115.5 47.5) (end 121 42) (width 0.2) (layer "B.Cu") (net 1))
 (segment (start 148.629 38.601) (end 200 38.601) (width 0.2) (layer "B.Cu") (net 1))
 (segment (start 112.5 49.565) (end 112.5 47.5) (width 0.2) (layer "B.Cu") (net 1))
 (segment (start 132.23 40.73) (end 139.365 40.73) (width 0.2) (layer "B.Cu") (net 1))
 (segment (start 205.0875 43.6885) (end 207.62 43.6885) (width 0.2) (layer "B.Cu") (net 1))
 (segment (start 146.5 40.73) (end 148.629 38.601) (width 0.2) (layer "B.Cu") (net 1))
 (segment (start 129.23 40.73) (end 132.23 40.73) (width 0.2) (layer "B.Cu") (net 1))
 (segment (start 112.5 47.5) (end 115.5 47.5) (width 0.2) (layer "B.Cu") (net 1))
 (segment (start 147.27 42.5) (end 146.5 43.27) (width 0.2) (layer "F.Cu") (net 2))
 (segment (start 179.05 45.08) (end 176.47 42.5) (width 0.2) (layer "F.Cu") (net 2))
 (segment (start 176.47 42.5) (end 147.27 42.5) (width 0.2) (layer "F.Cu") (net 2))
 (segment (start 183.1 45.08) (end 180.089 42.069) (width 0.2) (layer "F.Cu") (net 8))
 (segment (start 180.089 42.069) (end 140.566 42.069) (width 0.2) (layer "F.Cu") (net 8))
 (segment (start 140.566 42.069) (end 139.365 43.27) (width 0.2) (layer "F.Cu") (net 8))
 (segment (start 117 40.898834) (end 117 40.5) (width 0.2) (layer "F.Cu") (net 23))
 (segment (start 168.04 48) (end 124.101166 48) (width 0.2) (layer "F.Cu") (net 23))
 (segment (start 171 45.04) (end 168.04 48) (width 0.2) (layer "F.Cu") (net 23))
 (segment (start 124.101166 48) (end 117 40.898834) (width 0.2) (layer "F.Cu") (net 23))
 (segment (start 119 40.5) (end 120.899 38.601) (width 0.2) (layer "F.Cu") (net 20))
 (segment (start 197.4525 38.601) (end 207.62 48.7685) (width 0.2) (layer "F.Cu") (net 20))
 (segment (start 120.899 38.601) (end 197.4525 38.601) (width 0.2) (layer "F.Cu") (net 20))
 (segment (start 181.322872 48.7685) (end 192.38 48.7685) (width 0.2) (layer "B.Cu") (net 13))
 (segment (start 175 42.445628) (end 181.322872 48.7685) (width 0.2) (layer "B.Cu") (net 13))
 (segment (start 175 40) (end 175 42.445628) (width 0.2) (layer "B.Cu") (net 13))
 (segment (start 179.05 43) (end 179.05 40) (width 0.2) (layer "B.Cu") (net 7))
 (segment (start 182.2785 46.2285) (end 182.275 46.225) (width 0.2) (layer "B.Cu") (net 7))
 (segment (start 182.275 46.225) (end 179.05 43) (width 0.2) (layer "B.Cu") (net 7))
 (segment (start 192.38 46.2285) (end 182.2785 46.2285) (width 0.2) (layer "B.Cu") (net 7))
 (segment (start 192.1915 43.5) (end 192.38 43.6885) (width 0.2) (layer "B.Cu") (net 9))
 (segment (start 186.6 43.5) (end 192.1915 43.5) (width 0.2) (layer "B.Cu") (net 9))
 (segment (start 183.1 40) (end 186.6 43.5) (width 0.2) (layer "B.Cu") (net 9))
 (segment (start 171 39.96) (end 173 41.96) (width 0.2) (layer "B.Cu") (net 12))
 (segment (start 179.125 51.625) (end 184.56 51.625) (width 0.2) (layer "B.Cu") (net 12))
 (segment (start 173 41.96) (end 173 45.5) (width 0.2) (layer "B.Cu") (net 12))
 (segment (start 173 45.5) (end 179.125 51.625) (width 0.2) (layer "B.Cu") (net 12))
 (segment (start 203.8485 50) (end 207.62 46.2285) (width 0.2) (layer "B.Cu") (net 12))
 (segment (start 186.185 50) (end 203.8485 50) (width 0.2) (layer "B.Cu") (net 12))
 (segment (start 184.56 51.625) (end 186.185 50) (width 0.2) (layer "B.Cu") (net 12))
 (segment (start 191.3515 41.1485) (end 192.38 41.1485) (width 0.2) (layer "F.Cu") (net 11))
 (segment (start 114.56 49.125) (end 183.375 49.125) (width 0.2) (layer "F.Cu") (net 11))
 (segment (start 183.375 49.125) (end 191.3515 41.1485) (width 0.2) (layer "F.Cu") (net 11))
 (segment (start 124.49 65.6) (end 123.21 64.32) (width 0.2) (layer "B.Cu") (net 3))
 (segment (start 163.216667 64.72) (end 162.036667 64.72) (width 0.2) (layer "B.Cu") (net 3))
 (segment (start 209 61) (end 191 61) (width 0.2) (layer "B.Cu") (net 3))
 (segment (start 210.5 59.5) (end 209 61) (width 0.2) (layer "B.Cu") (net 3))
 (segment (start 132 80) (end 171 80) (width 0.2) (layer "B.Cu") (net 3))
 (segment (start 127.05 68.16) (end 124.49 65.6) (width 0.2) (layer "B.Cu") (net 3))
 (segment (start 167.056667 72.34) (end 167.056667 76.056667) (width 0.2) (layer "B.Cu") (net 3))
 (segment (start 207.62 53.8485) (end 208.8485 53.8485) (width 0.2) (layer "B.Cu") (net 3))
 (segment (start 208.8485 53.8485) (end 210.5 55.5) (width 0.2) (layer "B.Cu") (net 3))
 (segment (start 167.056667 76.056667) (end 171 80) (width 0.2) (layer "B.Cu") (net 3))
 (segment (start 191 61) (end 190 62) (width 0.2) (layer "B.Cu") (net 3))
 (segment (start 167.056667 72.34) (end 167.056667 68.56) (width 0.2) (layer "B.Cu") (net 3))
 (segment (start 123.21 64.32) (end 122.03 64.32) (width 0.2) (layer "B.Cu") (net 3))
 (segment (start 190 77.5) (end 187.5 80) (width 0.2) (layer "B.Cu") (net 3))
 (segment (start 127.05 71.94) (end 127.05 75.05) (width 0.2) (layer "B.Cu") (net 3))
 (segment (start 164.496667 66) (end 163.216667 64.72) (width 0.2) (layer "B.Cu") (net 3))
 (segment (start 190 62) (end 190 77.5) (width 0.2) (layer "B.Cu") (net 3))
 (segment (start 127.05 71.94) (end 127.05 68.16) (width 0.2) (layer "B.Cu") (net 3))
 (segment (start 127.05 75.05) (end 132 80) (width 0.2) (layer "B.Cu") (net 3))
 (segment (start 167.056667 68.56) (end 164.496667 66) (width 0.2) (layer "B.Cu") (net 3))
 (segment (start 171 80) (end 187.5 80) (width 0.2) (layer "B.Cu") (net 3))
 (segment (start 210.5 55.5) (end 210.5 59.5) (width 0.2) (layer "B.Cu") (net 3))
 (segment (start 184.5 66.2) (end 199.3915 51.3085) (width 0.2) (layer "F.Cu") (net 5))
 (segment (start 182.04 64.92) (end 182.04 64.77748) (width 0.2) (layer "F.Cu") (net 5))
 (segment (start 145.053333 61.5) (end 142.033333 64.52) (width 0.2) (layer "F.Cu") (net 5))
 (segment (start 182.04 64.77748) (end 178.76252 61.5) (width 0.2) (layer "F.Cu") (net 5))
 (segment (start 178.76252 61.5) (end 145.053333 61.5) (width 0.2) (layer "F.Cu") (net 5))
 (segment (start 199.3915 51.3085) (end 207.62 51.3085) (width 0.2) (layer "F.Cu") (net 5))
 (segment (start 143.313333 65.8) (end 144.493333 65.8) (width 0.2) (layer "B.Cu") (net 5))
 (segment (start 183.22 64.92) (end 182.04 64.92) (width 0.2) (layer "B.Cu") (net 5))
 (segment (start 184.5 66.2) (end 183.22 64.92) (width 0.2) (layer "B.Cu") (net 5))
 (segment (start 142.033333 64.52) (end 143.313333 65.8) (width 0.2) (layer "B.Cu") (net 5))
 (segment (start 147.053333 68.36) (end 147.053333 72.14) (width 0.2) (layer "B.Cu") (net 5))
 (segment (start 187.06 68.76) (end 184.5 66.2) (width 0.2) (layer "B.Cu") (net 5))
 (segment (start 144.493333 65.8) (end 147.053333 68.36) (width 0.2) (layer "B.Cu") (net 5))
 (segment (start 187.06 72.54) (end 187.06 68.76) (width 0.2) (layer "B.Cu") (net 5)))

